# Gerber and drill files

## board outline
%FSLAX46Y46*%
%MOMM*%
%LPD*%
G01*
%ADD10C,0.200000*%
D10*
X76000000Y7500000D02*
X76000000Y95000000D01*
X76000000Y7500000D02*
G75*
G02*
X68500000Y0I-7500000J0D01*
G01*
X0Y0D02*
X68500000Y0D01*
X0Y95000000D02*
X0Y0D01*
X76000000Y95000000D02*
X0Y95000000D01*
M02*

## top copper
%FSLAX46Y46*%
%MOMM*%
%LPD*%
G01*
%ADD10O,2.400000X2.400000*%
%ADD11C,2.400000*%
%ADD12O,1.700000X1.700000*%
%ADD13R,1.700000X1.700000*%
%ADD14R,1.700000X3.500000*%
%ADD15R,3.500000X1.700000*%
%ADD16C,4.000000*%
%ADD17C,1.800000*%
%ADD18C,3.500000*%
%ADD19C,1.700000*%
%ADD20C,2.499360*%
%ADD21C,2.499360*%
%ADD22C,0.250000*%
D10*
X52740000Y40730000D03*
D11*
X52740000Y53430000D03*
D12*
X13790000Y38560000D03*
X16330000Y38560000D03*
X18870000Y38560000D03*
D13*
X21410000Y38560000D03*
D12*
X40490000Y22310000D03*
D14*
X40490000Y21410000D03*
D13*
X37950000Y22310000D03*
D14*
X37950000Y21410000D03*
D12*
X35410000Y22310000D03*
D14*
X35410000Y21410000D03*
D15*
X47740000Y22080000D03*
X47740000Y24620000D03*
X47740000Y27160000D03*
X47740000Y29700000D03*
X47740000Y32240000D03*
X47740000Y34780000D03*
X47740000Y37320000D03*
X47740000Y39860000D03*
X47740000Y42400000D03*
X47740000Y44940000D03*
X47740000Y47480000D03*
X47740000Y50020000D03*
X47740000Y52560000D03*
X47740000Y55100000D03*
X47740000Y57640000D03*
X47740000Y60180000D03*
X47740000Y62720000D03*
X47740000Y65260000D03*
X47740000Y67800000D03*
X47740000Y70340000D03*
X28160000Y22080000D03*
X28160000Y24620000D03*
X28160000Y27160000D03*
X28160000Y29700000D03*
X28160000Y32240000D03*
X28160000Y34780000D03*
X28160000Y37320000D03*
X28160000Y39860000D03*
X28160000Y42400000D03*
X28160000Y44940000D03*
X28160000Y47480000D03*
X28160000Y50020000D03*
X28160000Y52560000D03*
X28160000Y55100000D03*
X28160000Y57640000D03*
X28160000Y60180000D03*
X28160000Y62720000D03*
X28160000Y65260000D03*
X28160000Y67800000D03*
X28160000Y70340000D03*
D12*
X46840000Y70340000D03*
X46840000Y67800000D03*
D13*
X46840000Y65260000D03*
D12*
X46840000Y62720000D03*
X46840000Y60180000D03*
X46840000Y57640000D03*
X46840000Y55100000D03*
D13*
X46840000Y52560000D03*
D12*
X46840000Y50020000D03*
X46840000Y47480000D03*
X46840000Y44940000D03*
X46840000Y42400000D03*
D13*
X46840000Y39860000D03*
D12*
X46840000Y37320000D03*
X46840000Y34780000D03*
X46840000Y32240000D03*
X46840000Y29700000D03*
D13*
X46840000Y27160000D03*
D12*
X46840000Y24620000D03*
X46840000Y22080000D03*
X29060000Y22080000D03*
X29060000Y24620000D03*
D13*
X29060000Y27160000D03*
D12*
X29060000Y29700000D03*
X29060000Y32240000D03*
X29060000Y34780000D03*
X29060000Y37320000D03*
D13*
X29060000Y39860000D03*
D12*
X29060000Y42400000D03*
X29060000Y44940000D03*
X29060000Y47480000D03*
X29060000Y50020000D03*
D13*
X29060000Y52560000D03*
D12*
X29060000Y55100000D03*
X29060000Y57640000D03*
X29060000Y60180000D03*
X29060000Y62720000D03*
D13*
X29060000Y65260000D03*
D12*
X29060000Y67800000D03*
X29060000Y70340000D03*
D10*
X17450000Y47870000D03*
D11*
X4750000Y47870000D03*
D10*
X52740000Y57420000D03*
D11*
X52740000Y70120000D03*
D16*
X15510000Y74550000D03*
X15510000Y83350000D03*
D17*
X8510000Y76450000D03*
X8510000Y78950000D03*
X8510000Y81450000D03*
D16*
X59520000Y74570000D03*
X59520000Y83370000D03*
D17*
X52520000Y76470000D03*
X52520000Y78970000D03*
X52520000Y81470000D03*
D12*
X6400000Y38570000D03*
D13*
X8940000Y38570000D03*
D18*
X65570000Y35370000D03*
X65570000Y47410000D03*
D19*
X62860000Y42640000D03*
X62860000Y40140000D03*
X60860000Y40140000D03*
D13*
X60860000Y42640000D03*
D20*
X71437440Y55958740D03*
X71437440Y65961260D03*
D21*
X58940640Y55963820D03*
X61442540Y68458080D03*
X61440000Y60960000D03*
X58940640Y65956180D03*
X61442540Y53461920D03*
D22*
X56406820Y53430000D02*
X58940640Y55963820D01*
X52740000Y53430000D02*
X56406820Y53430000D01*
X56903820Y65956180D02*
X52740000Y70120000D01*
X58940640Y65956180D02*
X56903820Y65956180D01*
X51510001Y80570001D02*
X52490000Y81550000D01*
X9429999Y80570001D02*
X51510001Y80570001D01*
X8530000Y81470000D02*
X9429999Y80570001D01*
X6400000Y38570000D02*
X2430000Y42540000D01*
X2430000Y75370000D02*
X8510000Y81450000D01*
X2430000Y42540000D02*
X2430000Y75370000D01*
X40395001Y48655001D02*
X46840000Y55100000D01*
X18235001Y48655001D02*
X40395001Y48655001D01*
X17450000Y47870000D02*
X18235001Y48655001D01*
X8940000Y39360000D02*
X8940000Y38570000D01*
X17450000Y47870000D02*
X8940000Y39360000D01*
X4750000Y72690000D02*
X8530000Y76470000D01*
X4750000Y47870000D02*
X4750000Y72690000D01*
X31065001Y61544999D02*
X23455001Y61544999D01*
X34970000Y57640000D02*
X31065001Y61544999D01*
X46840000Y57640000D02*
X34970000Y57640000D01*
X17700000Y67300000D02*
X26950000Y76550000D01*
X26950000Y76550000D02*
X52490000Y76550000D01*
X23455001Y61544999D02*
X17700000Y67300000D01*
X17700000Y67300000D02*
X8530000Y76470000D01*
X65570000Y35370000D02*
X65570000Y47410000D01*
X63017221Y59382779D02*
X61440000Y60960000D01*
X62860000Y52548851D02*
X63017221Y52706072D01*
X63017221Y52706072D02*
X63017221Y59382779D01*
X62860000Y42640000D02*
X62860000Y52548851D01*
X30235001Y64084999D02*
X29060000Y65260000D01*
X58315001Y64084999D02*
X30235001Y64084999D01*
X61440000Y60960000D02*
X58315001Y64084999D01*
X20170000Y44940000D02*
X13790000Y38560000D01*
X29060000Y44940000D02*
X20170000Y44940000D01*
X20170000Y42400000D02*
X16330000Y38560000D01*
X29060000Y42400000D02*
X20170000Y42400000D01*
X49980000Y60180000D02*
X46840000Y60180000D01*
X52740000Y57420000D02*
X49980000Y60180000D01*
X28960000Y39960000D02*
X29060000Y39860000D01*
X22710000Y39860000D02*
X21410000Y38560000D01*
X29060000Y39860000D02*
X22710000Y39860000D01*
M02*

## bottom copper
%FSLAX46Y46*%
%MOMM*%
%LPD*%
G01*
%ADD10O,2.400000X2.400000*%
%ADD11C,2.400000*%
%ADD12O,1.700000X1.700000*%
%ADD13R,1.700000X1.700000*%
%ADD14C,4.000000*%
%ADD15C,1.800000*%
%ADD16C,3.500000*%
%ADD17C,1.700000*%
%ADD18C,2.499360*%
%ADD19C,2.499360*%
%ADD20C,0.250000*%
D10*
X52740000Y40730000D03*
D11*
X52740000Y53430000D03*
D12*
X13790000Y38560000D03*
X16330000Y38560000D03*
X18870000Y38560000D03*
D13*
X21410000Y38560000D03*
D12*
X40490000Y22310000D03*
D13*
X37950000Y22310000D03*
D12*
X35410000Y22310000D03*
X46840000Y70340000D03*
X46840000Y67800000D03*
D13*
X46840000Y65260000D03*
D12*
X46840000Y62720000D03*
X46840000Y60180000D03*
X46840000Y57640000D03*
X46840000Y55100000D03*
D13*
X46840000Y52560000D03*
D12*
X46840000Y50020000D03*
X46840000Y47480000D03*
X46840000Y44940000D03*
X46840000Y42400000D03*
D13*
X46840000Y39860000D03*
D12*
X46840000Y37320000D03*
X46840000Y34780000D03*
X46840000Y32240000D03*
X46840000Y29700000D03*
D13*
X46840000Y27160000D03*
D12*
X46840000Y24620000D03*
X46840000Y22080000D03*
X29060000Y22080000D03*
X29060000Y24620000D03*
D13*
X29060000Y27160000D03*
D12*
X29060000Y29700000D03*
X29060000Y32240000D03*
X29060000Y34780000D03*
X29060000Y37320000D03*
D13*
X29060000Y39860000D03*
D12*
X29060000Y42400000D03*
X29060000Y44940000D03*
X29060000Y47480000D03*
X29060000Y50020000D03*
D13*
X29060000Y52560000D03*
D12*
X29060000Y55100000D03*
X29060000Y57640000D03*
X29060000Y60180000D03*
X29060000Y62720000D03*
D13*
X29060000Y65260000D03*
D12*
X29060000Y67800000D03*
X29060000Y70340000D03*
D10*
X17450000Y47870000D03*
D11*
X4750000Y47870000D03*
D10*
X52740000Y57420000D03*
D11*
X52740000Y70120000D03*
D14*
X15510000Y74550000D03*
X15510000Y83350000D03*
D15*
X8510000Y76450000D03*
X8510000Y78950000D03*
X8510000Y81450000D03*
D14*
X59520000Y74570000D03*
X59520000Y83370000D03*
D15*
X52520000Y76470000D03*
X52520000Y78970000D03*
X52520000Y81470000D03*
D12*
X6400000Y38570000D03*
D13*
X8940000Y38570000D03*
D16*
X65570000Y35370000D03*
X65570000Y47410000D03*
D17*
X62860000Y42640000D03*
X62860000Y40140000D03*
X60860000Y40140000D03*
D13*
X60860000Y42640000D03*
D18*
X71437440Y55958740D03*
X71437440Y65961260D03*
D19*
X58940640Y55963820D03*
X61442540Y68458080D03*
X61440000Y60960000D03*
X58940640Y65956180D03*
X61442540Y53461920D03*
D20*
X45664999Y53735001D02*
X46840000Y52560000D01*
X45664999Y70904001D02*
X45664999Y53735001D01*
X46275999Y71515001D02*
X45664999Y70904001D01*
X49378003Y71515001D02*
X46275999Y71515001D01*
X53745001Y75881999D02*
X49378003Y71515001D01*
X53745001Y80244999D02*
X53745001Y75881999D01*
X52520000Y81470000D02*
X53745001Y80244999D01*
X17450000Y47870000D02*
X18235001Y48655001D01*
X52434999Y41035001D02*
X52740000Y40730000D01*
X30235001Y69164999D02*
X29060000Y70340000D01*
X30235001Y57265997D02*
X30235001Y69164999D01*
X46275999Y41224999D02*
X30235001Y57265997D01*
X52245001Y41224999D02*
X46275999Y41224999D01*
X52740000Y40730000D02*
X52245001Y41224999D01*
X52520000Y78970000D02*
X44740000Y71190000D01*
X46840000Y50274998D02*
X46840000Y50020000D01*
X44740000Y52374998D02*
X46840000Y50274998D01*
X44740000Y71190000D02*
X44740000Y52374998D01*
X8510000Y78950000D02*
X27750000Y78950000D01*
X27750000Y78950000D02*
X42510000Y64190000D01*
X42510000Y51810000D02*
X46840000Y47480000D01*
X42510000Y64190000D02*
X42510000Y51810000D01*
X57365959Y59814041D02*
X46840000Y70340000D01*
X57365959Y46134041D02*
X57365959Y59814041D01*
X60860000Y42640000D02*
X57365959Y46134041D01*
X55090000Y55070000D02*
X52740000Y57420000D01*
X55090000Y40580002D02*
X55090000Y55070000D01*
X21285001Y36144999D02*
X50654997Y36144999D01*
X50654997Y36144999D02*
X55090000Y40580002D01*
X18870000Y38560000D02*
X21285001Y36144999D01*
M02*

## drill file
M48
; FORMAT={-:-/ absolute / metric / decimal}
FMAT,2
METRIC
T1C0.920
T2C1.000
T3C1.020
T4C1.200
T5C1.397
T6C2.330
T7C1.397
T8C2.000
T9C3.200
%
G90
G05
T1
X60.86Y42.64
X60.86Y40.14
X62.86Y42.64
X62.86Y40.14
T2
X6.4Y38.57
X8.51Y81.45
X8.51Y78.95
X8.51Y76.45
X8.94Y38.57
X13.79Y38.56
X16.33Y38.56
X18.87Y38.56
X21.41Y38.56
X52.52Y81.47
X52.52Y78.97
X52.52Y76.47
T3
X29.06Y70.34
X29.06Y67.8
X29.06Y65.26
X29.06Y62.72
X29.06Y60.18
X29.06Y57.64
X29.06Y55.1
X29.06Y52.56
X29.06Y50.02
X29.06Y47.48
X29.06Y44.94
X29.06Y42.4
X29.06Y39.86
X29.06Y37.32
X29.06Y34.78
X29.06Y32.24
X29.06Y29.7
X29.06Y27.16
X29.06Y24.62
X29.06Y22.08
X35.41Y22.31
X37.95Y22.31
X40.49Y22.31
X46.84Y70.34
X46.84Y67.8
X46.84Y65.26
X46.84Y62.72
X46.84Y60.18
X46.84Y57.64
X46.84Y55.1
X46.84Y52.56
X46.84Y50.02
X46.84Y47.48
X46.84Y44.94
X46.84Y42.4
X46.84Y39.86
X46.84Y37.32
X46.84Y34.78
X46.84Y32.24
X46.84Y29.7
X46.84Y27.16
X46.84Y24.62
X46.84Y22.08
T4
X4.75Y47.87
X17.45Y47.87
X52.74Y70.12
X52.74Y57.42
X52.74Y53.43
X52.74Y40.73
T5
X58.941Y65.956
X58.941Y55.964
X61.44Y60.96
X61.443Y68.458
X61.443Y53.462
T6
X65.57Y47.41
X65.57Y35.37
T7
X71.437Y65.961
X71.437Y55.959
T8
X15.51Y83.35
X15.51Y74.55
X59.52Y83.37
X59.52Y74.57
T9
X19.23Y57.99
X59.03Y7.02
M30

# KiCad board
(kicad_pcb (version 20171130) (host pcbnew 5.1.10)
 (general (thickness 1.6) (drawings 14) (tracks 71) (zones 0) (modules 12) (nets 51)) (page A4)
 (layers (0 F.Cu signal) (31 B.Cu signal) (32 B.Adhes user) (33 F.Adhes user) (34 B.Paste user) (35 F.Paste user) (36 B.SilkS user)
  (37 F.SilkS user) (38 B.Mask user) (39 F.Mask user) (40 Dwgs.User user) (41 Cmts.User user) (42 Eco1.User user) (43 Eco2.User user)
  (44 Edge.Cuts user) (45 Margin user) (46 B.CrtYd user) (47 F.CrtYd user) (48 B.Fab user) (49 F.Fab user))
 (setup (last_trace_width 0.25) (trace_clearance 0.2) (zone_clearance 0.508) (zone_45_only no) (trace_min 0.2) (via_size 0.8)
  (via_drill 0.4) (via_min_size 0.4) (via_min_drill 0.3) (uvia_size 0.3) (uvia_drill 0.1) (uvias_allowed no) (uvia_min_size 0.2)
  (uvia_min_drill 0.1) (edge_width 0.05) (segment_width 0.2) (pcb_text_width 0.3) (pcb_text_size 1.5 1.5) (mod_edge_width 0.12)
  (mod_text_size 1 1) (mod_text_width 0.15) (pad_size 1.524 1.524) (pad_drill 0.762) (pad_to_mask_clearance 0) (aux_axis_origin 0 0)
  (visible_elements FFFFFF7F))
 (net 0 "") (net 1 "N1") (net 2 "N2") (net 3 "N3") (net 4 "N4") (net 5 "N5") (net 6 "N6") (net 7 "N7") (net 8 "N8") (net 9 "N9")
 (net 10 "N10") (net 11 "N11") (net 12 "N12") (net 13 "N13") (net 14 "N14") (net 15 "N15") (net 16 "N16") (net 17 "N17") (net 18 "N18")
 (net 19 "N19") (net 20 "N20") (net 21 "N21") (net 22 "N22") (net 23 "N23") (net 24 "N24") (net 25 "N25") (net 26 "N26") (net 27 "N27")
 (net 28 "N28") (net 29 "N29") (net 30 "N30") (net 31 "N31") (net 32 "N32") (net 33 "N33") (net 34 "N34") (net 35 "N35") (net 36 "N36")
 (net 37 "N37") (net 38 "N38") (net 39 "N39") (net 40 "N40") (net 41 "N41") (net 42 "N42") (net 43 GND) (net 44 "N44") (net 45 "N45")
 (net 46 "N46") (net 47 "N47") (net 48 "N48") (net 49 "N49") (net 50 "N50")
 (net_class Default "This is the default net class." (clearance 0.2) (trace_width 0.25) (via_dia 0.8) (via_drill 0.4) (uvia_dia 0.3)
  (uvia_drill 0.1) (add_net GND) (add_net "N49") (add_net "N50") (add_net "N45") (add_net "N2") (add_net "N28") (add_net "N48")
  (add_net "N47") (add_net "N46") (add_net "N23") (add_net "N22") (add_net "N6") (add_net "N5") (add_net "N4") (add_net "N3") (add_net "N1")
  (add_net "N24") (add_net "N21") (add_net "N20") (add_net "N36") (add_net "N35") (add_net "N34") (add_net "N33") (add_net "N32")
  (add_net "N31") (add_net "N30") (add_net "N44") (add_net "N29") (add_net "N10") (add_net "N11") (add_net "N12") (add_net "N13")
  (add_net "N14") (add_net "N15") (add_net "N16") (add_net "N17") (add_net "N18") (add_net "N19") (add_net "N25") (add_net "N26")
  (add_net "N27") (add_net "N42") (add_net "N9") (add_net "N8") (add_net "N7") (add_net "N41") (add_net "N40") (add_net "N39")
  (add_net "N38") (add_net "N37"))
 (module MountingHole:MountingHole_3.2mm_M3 (layer F.Cu) (at 59.03 -7.02)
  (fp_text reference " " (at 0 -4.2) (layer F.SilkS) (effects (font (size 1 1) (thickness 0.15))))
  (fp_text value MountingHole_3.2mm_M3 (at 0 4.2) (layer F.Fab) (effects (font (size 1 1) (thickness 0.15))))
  (pad 1 np_thru_hole circle (at 0 0) (size 3.2 3.2) (drill 3.2) (layers *.Cu *.Mask)))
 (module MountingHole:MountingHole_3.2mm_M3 (layer F.Cu) (at 19.23 -57.99)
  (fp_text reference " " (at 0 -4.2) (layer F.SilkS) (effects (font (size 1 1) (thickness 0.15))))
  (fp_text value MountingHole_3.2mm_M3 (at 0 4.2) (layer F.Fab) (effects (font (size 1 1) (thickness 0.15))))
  (pad 1 np_thru_hole circle (at 0 0) (size 3.2 3.2) (drill 3.2) (layers *.Cu *.Mask)))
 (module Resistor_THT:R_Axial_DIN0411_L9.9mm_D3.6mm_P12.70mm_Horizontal (layer F.Cu) (at 52.74 -53.43 270)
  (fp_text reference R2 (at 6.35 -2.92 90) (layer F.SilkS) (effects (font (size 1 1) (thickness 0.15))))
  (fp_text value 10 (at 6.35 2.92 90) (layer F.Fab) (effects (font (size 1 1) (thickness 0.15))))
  (pad 2 thru_hole oval (at 12.7 0 270) (size 2.4 2.4) (drill 1.2) (layers *.Cu *.Mask) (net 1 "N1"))
  (pad 1 thru_hole circle (at 0 0 270) (size 2.4 2.4) (drill 1.2) (layers *.Cu *.Mask) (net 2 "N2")))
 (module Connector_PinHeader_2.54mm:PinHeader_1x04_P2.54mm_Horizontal (layer F.Cu) (at 21.41 -38.56 270)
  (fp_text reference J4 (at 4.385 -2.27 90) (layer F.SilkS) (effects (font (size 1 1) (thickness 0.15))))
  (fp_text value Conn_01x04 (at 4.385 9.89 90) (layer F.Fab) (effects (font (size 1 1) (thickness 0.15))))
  (pad 4 thru_hole oval (at 0 7.62 270) (size 1.7 1.7) (drill 1) (layers *.Cu *.Mask) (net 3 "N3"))
  (pad 3 thru_hole oval (at 0 5.08 270) (size 1.7 1.7) (drill 1) (layers *.Cu *.Mask) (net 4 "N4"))
  (pad 2 thru_hole oval (at 0 2.54 270) (size 1.7 1.7) (drill 1) (layers *.Cu *.Mask) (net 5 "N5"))
  (pad 1 thru_hole rect (at 0 0 270) (size 1.7 1.7) (drill 1) (layers *.Cu *.Mask) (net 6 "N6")))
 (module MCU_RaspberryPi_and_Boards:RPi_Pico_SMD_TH (layer F.Cu) (at 37.95 -46.21)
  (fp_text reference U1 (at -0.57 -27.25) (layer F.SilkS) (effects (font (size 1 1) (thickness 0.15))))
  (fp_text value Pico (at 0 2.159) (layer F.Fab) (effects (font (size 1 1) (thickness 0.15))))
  (pad 43 thru_hole oval (at 2.54 23.9) (size 1.7 1.7) (drill 1.02) (layers *.Cu *.Mask) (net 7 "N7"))
  (pad 43 smd rect (at 2.54 23.9 90) (size 3.5 1.7) (drill (offset -0.9 0)) (layers F.Cu F.Mask) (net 7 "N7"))
  (pad 42 thru_hole rect (at 0 23.9) (size 1.7 1.7) (drill 1.02) (layers *.Cu *.Mask) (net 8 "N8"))
  (pad 42 smd rect (at 0 23.9 90) (size 3.5 1.7) (drill (offset -0.9 0)) (layers F.Cu F.Mask) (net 8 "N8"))
  (pad 41 thru_hole oval (at -2.54 23.9) (size 1.7 1.7) (drill 1.02) (layers *.Cu *.Mask) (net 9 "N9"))
  (pad 41 smd rect (at -2.54 23.9 90) (size 3.5 1.7) (drill (offset -0.9 0)) (layers F.Cu F.Mask) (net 9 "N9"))
  (pad 21 smd rect (at 8.89 24.13) (size 3.5 1.7) (drill (offset 0.9 0)) (layers F.Cu F.Mask) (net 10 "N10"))
  (pad 22 smd rect (at 8.89 21.59) (size 3.5 1.7) (drill (offset 0.9 0)) (layers F.Cu F.Mask) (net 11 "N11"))
  (pad 23 smd rect (at 8.89 19.05) (size 3.5 1.7) (drill (offset 0.9 0)) (layers F.Cu F.Mask) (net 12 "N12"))
  (pad 24 smd rect (at 8.89 16.51) (size 3.5 1.7) (drill (offset 0.9 0)) (layers F.Cu F.Mask) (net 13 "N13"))
  (pad 25 smd rect (at 8.89 13.97) (size 3.5 1.7) (drill (offset 0.9 0)) (layers F.Cu F.Mask) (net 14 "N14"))
  (pad 26 smd rect (at 8.89 11.43) (size 3.5 1.7) (drill (offset 0.9 0)) (layers F.Cu F.Mask) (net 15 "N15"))
  (pad 27 smd rect (at 8.89 8.89) (size 3.5 1.7) (drill (offset 0.9 0)) (layers F.Cu F.Mask) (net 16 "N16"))
  (pad 28 smd rect (at 8.89 6.35) (size 3.5 1.7) (drill (offset 0.9 0)) (layers F.Cu F.Mask) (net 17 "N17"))
  (pad 29 smd rect (at 8.89 3.81) (size 3.5 1.7) (drill (offset 0.9 0)) (layers F.Cu F.Mask) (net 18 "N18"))
  (pad 30 smd rect (at 8.89 1.27) (size 3.5 1.7) (drill (offset 0.9 0)) (layers F.Cu F.Mask) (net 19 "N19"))
  (pad 31 smd rect (at 8.89 -1.27) (size 3.5 1.7) (drill (offset 0.9 0)) (layers F.Cu F.Mask) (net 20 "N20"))
  (pad 32 smd rect (at 8.89 -3.81) (size 3.5 1.7) (drill (offset 0.9 0)) (layers F.Cu F.Mask) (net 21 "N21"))
  (pad 33 smd rect (at 8.89 -6.35) (size 3.5 1.7) (drill (offset 0.9 0)) (layers F.Cu F.Mask) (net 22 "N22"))
  (pad 34 smd rect (at 8.89 -8.89) (size 3.5 1.7) (drill (offset 0.9 0)) (layers F.Cu F.Mask) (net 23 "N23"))
  (pad 35 smd rect (at 8.89 -11.43) (size 3.5 1.7) (drill (offset 0.9 0)) (layers F.Cu F.Mask) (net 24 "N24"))
  (pad 36 smd rect (at 8.89 -13.97) (size 3.5 1.7) (drill (offset 0.9 0)) (layers F.Cu F.Mask) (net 5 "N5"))
  (pad 37 smd rect (at 8.89 -16.51) (size 3.5 1.7) (drill (offset 0.9 0)) (layers F.Cu F.Mask) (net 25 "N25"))
  (pad 38 smd rect (at 8.89 -19.05) (size 3.5 1.7) (drill (offset 0.9 0)) (layers F.Cu F.Mask) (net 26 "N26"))
  (pad 39 smd rect (at 8.89 -21.59) (size 3.5 1.7) (drill (offset 0.9 0)) (layers F.Cu F.Mask) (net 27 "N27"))
  (pad 40 smd rect (at 8.89 -24.13) (size 3.5 1.7) (drill (offset 0.9 0)) (layers F.Cu F.Mask) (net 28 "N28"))
  (pad 20 smd rect (at -8.89 24.13) (size 3.5 1.7) (drill (offset -0.9 0)) (layers F.Cu F.Mask) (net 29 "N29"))
  (pad 19 smd rect (at -8.89 21.59) (size 3.5 1.7) (drill (offset -0.9 0)) (layers F.Cu F.Mask) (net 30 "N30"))
  (pad 18 smd rect (at -8.89 19.05) (size 3.5 1.7) (drill (offset -0.9 0)) (layers F.Cu F.Mask) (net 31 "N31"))
  (pad 17 smd rect (at -8.89 16.51) (size 3.5 1.7) (drill (offset -0.9 0)) (layers F.Cu F.Mask) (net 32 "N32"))
  (pad 16 smd rect (at -8.89 13.97) (size 3.5 1.7) (drill (offset -0.9 0)) (layers F.Cu F.Mask) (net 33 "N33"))
  (pad 15 smd rect (at -8.89 11.43) (size 3.5 1.7) (drill (offset -0.9 0)) (layers F.Cu F.Mask) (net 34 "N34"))
  (pad 14 smd rect (at -8.89 8.89) (size 3.5 1.7) (drill (offset -0.9 0)) (layers F.Cu F.Mask) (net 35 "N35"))
  (pad 13 smd rect (at -8.89 6.35) (size 3.5 1.7) (drill (offset -0.9 0)) (layers F.Cu F.Mask) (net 6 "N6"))
  (pad 12 smd rect (at -8.89 3.81) (size 3.5 1.7) (drill (offset -0.9 0)) (layers F.Cu F.Mask) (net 4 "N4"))
  (pad 11 smd rect (at -8.89 1.27) (size 3.5 1.7) (drill (offset -0.9 0)) (layers F.Cu F.Mask) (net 3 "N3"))
  (pad 10 smd rect (at -8.89 -1.27) (size 3.5 1.7) (drill (offset -0.9 0)) (layers F.Cu F.Mask) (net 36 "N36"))
  (pad 9 smd rect (at -8.89 -3.81) (size 3.5 1.7) (drill (offset -0.9 0)) (layers F.Cu F.Mask) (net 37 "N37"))
  (pad 8 smd rect (at -8.89 -6.35) (size 3.5 1.7) (drill (offset -0.9 0)) (layers F.Cu F.Mask) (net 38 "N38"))
  (pad 7 smd rect (at -8.89 -8.89) (size 3.5 1.7) (drill (offset -0.9 0)) (layers F.Cu F.Mask) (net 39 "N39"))
  (pad 6 smd rect (at -8.89 -11.43) (size 3.5 1.7) (drill (offset -0.9 0)) (layers F.Cu F.Mask) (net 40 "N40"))
  (pad 5 smd rect (at -8.89 -13.97) (size 3.5 1.7) (drill (offset -0.9 0)) (layers F.Cu F.Mask) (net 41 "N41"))
  (pad 4 smd rect (at -8.89 -16.51) (size 3.5 1.7) (drill (offset -0.9 0)) (layers F.Cu F.Mask) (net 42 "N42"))
  (pad 3 smd rect (at -8.89 -19.05) (size 3.5 1.7) (drill (offset -0.9 0)) (layers F.Cu F.Mask) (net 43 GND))
  (pad 2 smd rect (at -8.89 -21.59) (size 3.5 1.7) (drill (offset -0.9 0)) (layers F.Cu F.Mask) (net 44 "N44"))
  (pad 1 smd rect (at -8.89 -24.13) (size 3.5 1.7) (drill (offset -0.9 0)) (layers F.Cu F.Mask) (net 1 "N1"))
  (pad 40 thru_hole oval (at 8.89 -24.13) (size 1.7 1.7) (drill 1.02) (layers *.Cu *.Mask) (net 28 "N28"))
  (pad 39 thru_hole oval (at 8.89 -21.59) (size 1.7 1.7) (drill 1.02) (layers *.Cu *.Mask) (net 27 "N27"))
  (pad 38 thru_hole rect (at 8.89 -19.05) (size 1.7 1.7) (drill 1.02) (layers *.Cu *.Mask) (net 26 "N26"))
  (pad 37 thru_hole oval (at 8.89 -16.51) (size 1.7 1.7) (drill 1.02) (layers *.Cu *.Mask) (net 25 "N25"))
  (pad 36 thru_hole oval (at 8.89 -13.97) (size 1.7 1.7) (drill 1.02) (layers *.Cu *.Mask) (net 5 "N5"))
  (pad 35 thru_hole oval (at 8.89 -11.43) (size 1.7 1.7) (drill 1.02) (layers *.Cu *.Mask) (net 24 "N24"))
  (pad 34 thru_hole oval (at 8.89 -8.89) (size 1.7 1.7) (drill 1.02) (layers *.Cu *.Mask) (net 23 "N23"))
  (pad 33 thru_hole rect (at 8.89 -6.35) (size 1.7 1.7) (drill 1.02) (layers *.Cu *.Mask) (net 22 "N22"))
  (pad 32 thru_hole oval (at 8.89 -3.81) (size 1.7 1.7) (drill 1.02) (layers *.Cu *.Mask) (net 21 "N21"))
  (pad 31 thru_hole oval (at 8.89 -1.27) (size 1.7 1.7) (drill 1.02) (layers *.Cu *.Mask) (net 20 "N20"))
  (pad 30 thru_hole oval (at 8.89 1.27) (size 1.7 1.7) (drill 1.02) (layers *.Cu *.Mask) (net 19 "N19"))
  (pad 29 thru_hole oval (at 8.89 3.81) (size 1.7 1.7) (drill 1.02) (layers *.Cu *.Mask) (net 18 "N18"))
  (pad 28 thru_hole rect (at 8.89 6.35) (size 1.7 1.7) (drill 1.02) (layers *.Cu *.Mask) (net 17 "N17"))
  (pad 27 thru_hole oval (at 8.89 8.89) (size 1.7 1.7) (drill 1.02) (layers *.Cu *.Mask) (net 16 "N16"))
  (pad 26 thru_hole oval (at 8.89 11.43) (size 1.7 1.7) (drill 1.02) (layers *.Cu *.Mask) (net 15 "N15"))
  (pad 25 thru_hole oval (at 8.89 13.97) (size 1.7 1.7) (drill 1.02) (layers *.Cu *.Mask) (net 14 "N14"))
  (pad 24 thru_hole oval (at 8.89 16.51) (size 1.7 1.7) (drill 1.02) (layers *.Cu *.Mask) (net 13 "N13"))
  (pad 23 thru_hole rect (at 8.89 19.05) (size 1.7 1.7) (drill 1.02) (layers *.Cu *.Mask) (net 12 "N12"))
  (pad 22 thru_hole oval (at 8.89 21.59) (size 1.7 1.7) (drill 1.02) (layers *.Cu *.Mask) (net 11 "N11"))
  (pad 21 thru_hole oval (at 8.89 24.13) (size 1.7 1.7) (drill 1.02) (layers *.Cu *.Mask) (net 10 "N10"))
  (pad 20 thru_hole oval (at -8.89 24.13) (size 1.7 1.7) (drill 1.02) (layers *.Cu *.Mask) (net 29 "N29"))
  (pad 19 thru_hole oval (at -8.89 21.59) (size 1.7 1.7) (drill 1.02) (layers *.Cu *.Mask) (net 30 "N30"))
  (pad 18 thru_hole rect (at -8.89 19.05) (size 1.7 1.7) (drill 1.02) (layers *.Cu *.Mask) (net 31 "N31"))
  (pad 17 thru_hole oval (at -8.89 16.51) (size 1.7 1.7) (drill 1.02) (layers *.Cu *.Mask) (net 32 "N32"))
  (pad 16 thru_hole oval (at -8.89 13.97) (size 1.7 1.7) (drill 1.02) (layers *.Cu *.Mask) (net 33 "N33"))
  (pad 15 thru_hole oval (at -8.89 11.43) (size 1.7 1.7) (drill 1.02) (layers *.Cu *.Mask) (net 34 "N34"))
  (pad 14 thru_hole oval (at -8.89 8.89) (size 1.7 1.7) (drill 1.02) (layers *.Cu *.Mask) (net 35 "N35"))
  (pad 13 thru_hole rect (at -8.89 6.35) (size 1.7 1.7) (drill 1.02) (layers *.Cu *.Mask) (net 6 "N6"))
  (pad 12 thru_hole oval (at -8.89 3.81) (size 1.7 1.7) (drill 1.02) (layers *.Cu *.Mask) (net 4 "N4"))
  (pad 11 thru_hole oval (at -8.89 1.27) (size 1.7 1.7) (drill 1.02) (layers *.Cu *.Mask) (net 3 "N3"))
  (pad 10 thru_hole oval (at -8.89 -1.27) (size 1.7 1.7) (drill 1.02) (layers *.Cu *.Mask) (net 36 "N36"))
  (pad 9 thru_hole oval (at -8.89 -3.81) (size 1.7 1.7) (drill 1.02) (layers *.Cu *.Mask) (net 37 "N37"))
  (pad 8 thru_hole rect (at -8.89 -6.35) (size 1.7 1.7) (drill 1.02) (layers *.Cu *.Mask) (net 38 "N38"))
  (pad 7 thru_hole oval (at -8.89 -8.89) (size 1.7 1.7) (drill 1.02) (layers *.Cu *.Mask) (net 39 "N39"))
  (pad 6 thru_hole oval (at -8.89 -11.43) (size 1.7 1.7) (drill 1.02) (layers *.Cu *.Mask) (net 40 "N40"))
  (pad 5 thru_hole oval (at -8.89 -13.97) (size 1.7 1.7) (drill 1.02) (layers *.Cu *.Mask) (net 41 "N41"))
  (pad 4 thru_hole oval (at -8.89 -16.51) (size 1.7 1.7) (drill 1.02) (layers *.Cu *.Mask) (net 42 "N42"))
  (pad 3 thru_hole rect (at -8.89 -19.05) (size 1.7 1.7) (drill 1.02) (layers *.Cu *.Mask) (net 43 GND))
  (pad 2 thru_hole oval (at -8.89 -21.59) (size 1.7 1.7) (drill 1.02) (layers *.Cu *.Mask) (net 44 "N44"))
  (pad 1 thru_hole oval (at -8.89 -24.13) (size 1.7 1.7) (drill 1.02) (layers *.Cu *.Mask) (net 1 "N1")))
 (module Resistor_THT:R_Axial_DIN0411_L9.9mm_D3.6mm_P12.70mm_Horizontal (layer F.Cu) (at 4.75 -47.87)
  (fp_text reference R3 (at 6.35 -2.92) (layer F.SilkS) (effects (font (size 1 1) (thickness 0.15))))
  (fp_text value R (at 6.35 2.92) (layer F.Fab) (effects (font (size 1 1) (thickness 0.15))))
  (pad 2 thru_hole oval (at 12.7 0) (size 2.4 2.4) (drill 1.2) (layers *.Cu *.Mask) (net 23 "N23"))
  (pad 1 thru_hole circle (at 0 0) (size 2.4 2.4) (drill 1.2) (layers *.Cu *.Mask) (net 24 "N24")))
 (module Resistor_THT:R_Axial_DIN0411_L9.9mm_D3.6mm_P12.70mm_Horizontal (layer F.Cu) (at 52.74 -70.12 270)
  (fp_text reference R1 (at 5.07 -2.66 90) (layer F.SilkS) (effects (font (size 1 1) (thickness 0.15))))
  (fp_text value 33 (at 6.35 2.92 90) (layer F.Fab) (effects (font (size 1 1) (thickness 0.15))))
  (pad 2 thru_hole oval (at 12.7 0 270) (size 2.4 2.4) (drill 1.2) (layers *.Cu *.Mask) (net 5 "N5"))
  (pad 1 thru_hole circle (at 0 0 270) (size 2.4 2.4) (drill 1.2) (layers *.Cu *.Mask) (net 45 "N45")))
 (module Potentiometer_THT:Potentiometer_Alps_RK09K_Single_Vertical (layer F.Cu) (at 8.51 -76.45)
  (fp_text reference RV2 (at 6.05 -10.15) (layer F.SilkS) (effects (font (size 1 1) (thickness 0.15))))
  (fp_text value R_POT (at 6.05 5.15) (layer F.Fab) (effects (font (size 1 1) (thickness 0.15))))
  (pad "" np_thru_hole circle (at 7 1.9) (size 4 4) (drill 2) (layers *.Cu *.Mask))
  (pad "" np_thru_hole circle (at 7 -6.9) (size 4 4) (drill 2) (layers *.Cu *.Mask))
  (pad 1 thru_hole circle (at 0 0) (size 1.8 1.8) (drill 1) (layers *.Cu *.Mask) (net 24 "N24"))
  (pad 2 thru_hole circle (at 0 -2.5) (size 1.8 1.8) (drill 1) (layers *.Cu *.Mask) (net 20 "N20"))
  (pad 3 thru_hole circle (at 0 -5) (size 1.8 1.8) (drill 1) (layers *.Cu *.Mask) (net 22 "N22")))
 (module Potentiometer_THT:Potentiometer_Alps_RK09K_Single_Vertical (layer F.Cu) (at 52.52 -76.47)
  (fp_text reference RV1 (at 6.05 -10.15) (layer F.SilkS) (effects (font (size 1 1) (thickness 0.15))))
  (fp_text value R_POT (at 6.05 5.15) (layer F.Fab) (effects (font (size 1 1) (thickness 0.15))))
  (pad "" np_thru_hole circle (at 7 1.9) (size 4 4) (drill 2) (layers *.Cu *.Mask))
  (pad "" np_thru_hole circle (at 7 -6.9) (size 4 4) (drill 2) (layers *.Cu *.Mask))
  (pad 1 thru_hole circle (at 0 0) (size 1.8 1.8) (drill 1) (layers *.Cu *.Mask) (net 24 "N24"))
  (pad 2 thru_hole circle (at 0 -2.5) (size 1.8 1.8) (drill 1) (layers *.Cu *.Mask) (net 21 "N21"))
  (pad 3 thru_hole circle (at 0 -5) (size 1.8 1.8) (drill 1) (layers *.Cu *.Mask) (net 22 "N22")))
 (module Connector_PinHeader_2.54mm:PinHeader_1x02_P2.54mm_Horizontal (layer F.Cu) (at 8.94 -38.57 270)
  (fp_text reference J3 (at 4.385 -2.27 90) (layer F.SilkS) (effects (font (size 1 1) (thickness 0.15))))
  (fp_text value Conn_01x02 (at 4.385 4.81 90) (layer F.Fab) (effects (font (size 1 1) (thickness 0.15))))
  (pad 2 thru_hole oval (at 0 2.54 270) (size 1.7 1.7) (drill 1) (layers *.Cu *.Mask) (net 22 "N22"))
  (pad 1 thru_hole rect (at 0 0 270) (size 1.7 1.7) (drill 1) (layers *.Cu *.Mask) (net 23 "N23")))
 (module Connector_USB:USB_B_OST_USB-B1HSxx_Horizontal (layer F.Cu) (at 60.86 -42.64)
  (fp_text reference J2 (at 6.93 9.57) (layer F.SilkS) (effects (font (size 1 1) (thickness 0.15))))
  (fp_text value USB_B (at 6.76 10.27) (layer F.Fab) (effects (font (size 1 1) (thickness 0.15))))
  (pad 5 thru_hole circle (at 4.71 7.27) (size 3.5 3.5) (drill 2.33) (layers *.Cu *.Mask) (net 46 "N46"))
  (pad 5 thru_hole circle (at 4.71 -4.77) (size 3.5 3.5) (drill 2.33) (layers *.Cu *.Mask) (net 46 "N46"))
  (pad 4 thru_hole circle (at 2 0) (size 1.7 1.7) (drill 0.92) (layers *.Cu *.Mask) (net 43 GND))
  (pad 3 thru_hole circle (at 2 2.5) (size 1.7 1.7) (drill 0.92) (layers *.Cu *.Mask) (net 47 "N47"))
  (pad 2 thru_hole circle (at 0 2.5) (size 1.7 1.7) (drill 0.92) (layers *.Cu *.Mask) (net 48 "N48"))
  (pad 1 thru_hole rect (at 0 0) (size 1.7 1.7) (drill 0.92) (layers *.Cu *.Mask) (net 28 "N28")))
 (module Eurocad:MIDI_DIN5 (layer F.Cu) (at 64.43974 -60.96 90)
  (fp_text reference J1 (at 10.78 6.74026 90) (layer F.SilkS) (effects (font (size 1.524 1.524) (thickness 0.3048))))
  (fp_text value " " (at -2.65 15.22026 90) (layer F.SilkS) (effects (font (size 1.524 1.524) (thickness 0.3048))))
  (pad "" np_thru_hole circle (at -5.00126 6.9977 90) (size 2.49936 2.49936) (drill 1.397) (layers *.Cu *.Mask F.SilkS))
  (pad "" np_thru_hole circle (at 5.00126 6.9977 90) (size 2.49936 2.49936) (drill 1.397) (layers *.Cu *.Mask F.SilkS))
  (pad 5 thru_hole circle (at -4.99618 -5.4991 90) (size 2.49936 2.49936) (drill 1.397) (layers *.Cu *.SilkS *.Mask) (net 2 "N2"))
  (pad 1 thru_hole circle (at 7.49808 -2.9972 90) (size 2.49936 2.49936) (drill 1.397) (layers *.Cu *.SilkS *.Mask) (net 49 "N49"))
  (pad 2 thru_hole circle (at 0 -2.99974 90) (size 2.49936 2.49936) (drill 1.397) (layers *.Cu *.SilkS *.Mask) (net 43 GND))
  (pad 4 thru_hole circle (at 4.99618 -5.4991 90) (size 2.49936 2.49936) (drill 1.397) (layers *.Cu *.SilkS *.Mask) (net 45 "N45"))
  (pad 3 thru_hole circle (at -7.49808 -2.9972 90) (size 2.49936 2.49936) (drill 1.397) (layers *.Cu *.SilkS *.Mask) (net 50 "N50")))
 (gr_line (start 76 -7.5) (end 76 -95) (layer Edge.Cuts) (width 0.2))
 (gr_arc (start 68.5 -7.5) (end 68.5 0) (angle -90) (layer Edge.Cuts) (width 0.2))
 (gr_line (start 0 0) (end 68.5 0) (layer Edge.Cuts) (width 0.2))
 (gr_line (start 0 -95) (end 0 0) (layer Edge.Cuts) (width 0.2))
 (gr_line (start 76 -95) (end 0 -95) (layer Edge.Cuts) (width 0.2))
 (segment (start 56.40682 -53.43) (end 58.94064 -55.96382) (width 0.25) (layer F.Cu) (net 2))
 (segment (start 52.74 -53.43) (end 56.40682 -53.43) (width 0.25) (layer F.Cu) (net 2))
 (segment (start 56.90382 -65.95618) (end 52.74 -70.12) (width 0.25) (layer F.Cu) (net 45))
 (segment (start 58.94064 -65.95618) (end 56.90382 -65.95618) (width 0.25) (layer F.Cu) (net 45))
 (segment (start 51.510001 -80.570001) (end 52.49 -81.55) (width 0.25) (layer F.Cu) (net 22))
 (segment (start 9.429999 -80.570001) (end 51.510001 -80.570001) (width 0.25) (layer F.Cu) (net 22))
 (segment (start 8.53 -81.47) (end 9.429999 -80.570001) (width 0.25) (layer F.Cu) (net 22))
 (segment (start 6.4 -38.57) (end 2.43 -42.54) (width 0.25) (layer F.Cu) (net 22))
 (segment (start 2.43 -75.37) (end 8.51 -81.45) (width 0.25) (layer F.Cu) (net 22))
 (segment (start 2.43 -42.54) (end 2.43 -75.37) (width 0.25) (layer F.Cu) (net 22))
 (segment (start 45.664999 -53.735001) (end 46.84 -52.56) (width 0.25) (layer B.Cu) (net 22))
 (segment (start 45.664999 -70.904001) (end 45.664999 -53.735001) (width 0.25) (layer B.Cu) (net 22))
 (segment (start 46.275999 -71.515001) (end 45.664999 -70.904001) (width 0.25) (layer B.Cu) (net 22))
 (segment (start 49.378003 -71.515001) (end 46.275999 -71.515001) (width 0.25) (layer B.Cu) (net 22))
 (segment (start 53.745001 -75.881999) (end 49.378003 -71.515001) (width 0.25) (layer B.Cu) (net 22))
 (segment (start 53.745001 -80.244999) (end 53.745001 -75.881999) (width 0.25) (layer B.Cu) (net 22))
 (segment (start 52.52 -81.47) (end 53.745001 -80.244999) (width 0.25) (layer B.Cu) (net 22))
 (segment (start 17.45 -47.87) (end 18.235001 -48.655001) (width 0.25) (layer B.Cu) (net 23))
 (segment (start 40.395001 -48.655001) (end 46.84 -55.1) (width 0.25) (layer F.Cu) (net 23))
 (segment (start 18.235001 -48.655001) (end 40.395001 -48.655001) (width 0.25) (layer F.Cu) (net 23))
 (segment (start 17.45 -47.87) (end 18.235001 -48.655001) (width 0.25) (layer F.Cu) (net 23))
 (segment (start 8.94 -39.36) (end 8.94 -38.57) (width 0.25) (layer F.Cu) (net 23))
 (segment (start 17.45 -47.87) (end 8.94 -39.36) (width 0.25) (layer F.Cu) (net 23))
 (segment (start 52.434999 -41.035001) (end 52.74 -40.73) (width 0.25) (layer B.Cu) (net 1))
 (segment (start 30.235001 -69.164999) (end 29.06 -70.34) (width 0.25) (layer B.Cu) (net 1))
 (segment (start 30.235001 -57.265997) (end 30.235001 -69.164999) (width 0.25) (layer B.Cu) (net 1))
 (segment (start 46.275999 -41.224999) (end 30.235001 -57.265997) (width 0.25) (layer B.Cu) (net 1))
 (segment (start 52.245001 -41.224999) (end 46.275999 -41.224999) (width 0.25) (layer B.Cu) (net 1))
 (segment (start 52.74 -40.73) (end 52.245001 -41.224999) (width 0.25) (layer B.Cu) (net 1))
 (segment (start 4.75 -72.69) (end 8.53 -76.47) (width 0.25) (layer F.Cu) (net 24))
 (segment (start 4.75 -47.87) (end 4.75 -72.69) (width 0.25) (layer F.Cu) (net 24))
 (segment (start 31.065001 -61.544999) (end 23.455001 -61.544999) (width 0.25) (layer F.Cu) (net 24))
 (segment (start 34.97 -57.64) (end 31.065001 -61.544999) (width 0.25) (layer F.Cu) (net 24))
 (segment (start 46.84 -57.64) (end 34.97 -57.64) (width 0.25) (layer F.Cu) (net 24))
 (segment (start 17.7 -67.3) (end 26.95 -76.55) (width 0.25) (layer F.Cu) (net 24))
 (segment (start 26.95 -76.55) (end 52.49 -76.55) (width 0.25) (layer F.Cu) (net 24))
 (segment (start 23.455001 -61.544999) (end 17.7 -67.3) (width 0.25) (layer F.Cu) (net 24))
 (segment (start 17.7 -67.3) (end 8.53 -76.47) (width 0.25) (layer F.Cu) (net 24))
 (segment (start 52.52 -78.97) (end 44.74 -71.19) (width 0.25) (layer B.Cu) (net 21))
 (segment (start 46.84 -50.274998) (end 46.84 -50.02) (width 0.25) (layer B.Cu) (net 21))
 (segment (start 44.74 -52.374998) (end 46.84 -50.274998) (width 0.25) (layer B.Cu) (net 21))
 (segment (start 44.74 -71.19) (end 44.74 -52.374998) (width 0.25) (layer B.Cu) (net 21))
 (segment (start 8.51 -78.95) (end 27.75 -78.95) (width 0.25) (layer B.Cu) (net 20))
 (segment (start 27.75 -78.95) (end 42.51 -64.19) (width 0.25) (layer B.Cu) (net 20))
 (segment (start 42.51 -51.81) (end 46.84 -47.48) (width 0.25) (layer B.Cu) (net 20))
 (segment (start 42.51 -64.19) (end 42.51 -51.81) (width 0.25) (layer B.Cu) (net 20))
 (segment (start 65.57 -35.37) (end 65.57 -47.41) (width 0.25) (layer F.Cu) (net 46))
 (segment (start 63.017221 -59.382779) (end 61.44 -60.96) (width 0.25) (layer F.Cu) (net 43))
 (segment (start 62.86 -52.548851) (end 63.017221 -52.706072) (width 0.25) (layer F.Cu) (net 43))
 (segment (start 63.017221 -52.706072) (end 63.017221 -59.382779) (width 0.25) (layer F.Cu) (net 43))
 (segment (start 62.86 -42.64) (end 62.86 -52.548851) (width 0.25) (layer F.Cu) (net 43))
 (segment (start 30.235001 -64.084999) (end 29.06 -65.26) (width 0.25) (layer F.Cu) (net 43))
 (segment (start 58.315001 -64.084999) (end 30.235001 -64.084999) (width 0.25) (layer F.Cu) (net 43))
 (segment (start 61.44 -60.96) (end 58.315001 -64.084999) (width 0.25) (layer F.Cu) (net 43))
 (segment (start 57.365959 -59.814041) (end 46.84 -70.34) (width 0.25) (layer B.Cu) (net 28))
 (segment (start 57.365959 -46.134041) (end 57.365959 -59.814041) (width 0.25) (layer B.Cu) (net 28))
 (segment (start 60.86 -42.64) (end 57.365959 -46.134041) (width 0.25) (layer B.Cu) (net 28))
 (segment (start 20.17 -44.94) (end 13.79 -38.56) (width 0.25) (layer F.Cu) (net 3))
 (segment (start 29.06 -44.94) (end 20.17 -44.94) (width 0.25) (layer F.Cu) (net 3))
 (segment (start 20.17 -42.4) (end 16.33 -38.56) (width 0.25) (layer F.Cu) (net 4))
 (segment (start 29.06 -42.4) (end 20.17 -42.4) (width 0.25) (layer F.Cu) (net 4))
 (segment (start 49.98 -60.18) (end 46.84 -60.18) (width 0.25) (layer F.Cu) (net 5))
 (segment (start 52.74 -57.42) (end 49.98 -60.18) (width 0.25) (layer F.Cu) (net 5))
 (segment (start 55.09 -55.07) (end 52.74 -57.42) (width 0.25) (layer B.Cu) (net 5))
 (segment (start 55.09 -40.580002) (end 55.09 -55.07) (width 0.25) (layer B.Cu) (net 5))
 (segment (start 21.285001 -36.144999) (end 50.654997 -36.144999) (width 0.25) (layer B.Cu) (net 5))
 (segment (start 50.654997 -36.144999) (end 55.09 -40.580002) (width 0.25) (layer B.Cu) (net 5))
 (segment (start 18.87 -38.56) (end 21.285001 -36.144999) (width 0.25) (layer B.Cu) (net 5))
 (segment (start 28.96 -39.96) (end 29.06 -39.86) (width 0.25) (layer F.Cu) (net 6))
 (segment (start 22.71 -39.86) (end 21.41 -38.56) (width 0.25) (layer F.Cu) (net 6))
 (segment (start 29.06 -39.86) (end 22.71 -39.86) (width 0.25) (layer F.Cu) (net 6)))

